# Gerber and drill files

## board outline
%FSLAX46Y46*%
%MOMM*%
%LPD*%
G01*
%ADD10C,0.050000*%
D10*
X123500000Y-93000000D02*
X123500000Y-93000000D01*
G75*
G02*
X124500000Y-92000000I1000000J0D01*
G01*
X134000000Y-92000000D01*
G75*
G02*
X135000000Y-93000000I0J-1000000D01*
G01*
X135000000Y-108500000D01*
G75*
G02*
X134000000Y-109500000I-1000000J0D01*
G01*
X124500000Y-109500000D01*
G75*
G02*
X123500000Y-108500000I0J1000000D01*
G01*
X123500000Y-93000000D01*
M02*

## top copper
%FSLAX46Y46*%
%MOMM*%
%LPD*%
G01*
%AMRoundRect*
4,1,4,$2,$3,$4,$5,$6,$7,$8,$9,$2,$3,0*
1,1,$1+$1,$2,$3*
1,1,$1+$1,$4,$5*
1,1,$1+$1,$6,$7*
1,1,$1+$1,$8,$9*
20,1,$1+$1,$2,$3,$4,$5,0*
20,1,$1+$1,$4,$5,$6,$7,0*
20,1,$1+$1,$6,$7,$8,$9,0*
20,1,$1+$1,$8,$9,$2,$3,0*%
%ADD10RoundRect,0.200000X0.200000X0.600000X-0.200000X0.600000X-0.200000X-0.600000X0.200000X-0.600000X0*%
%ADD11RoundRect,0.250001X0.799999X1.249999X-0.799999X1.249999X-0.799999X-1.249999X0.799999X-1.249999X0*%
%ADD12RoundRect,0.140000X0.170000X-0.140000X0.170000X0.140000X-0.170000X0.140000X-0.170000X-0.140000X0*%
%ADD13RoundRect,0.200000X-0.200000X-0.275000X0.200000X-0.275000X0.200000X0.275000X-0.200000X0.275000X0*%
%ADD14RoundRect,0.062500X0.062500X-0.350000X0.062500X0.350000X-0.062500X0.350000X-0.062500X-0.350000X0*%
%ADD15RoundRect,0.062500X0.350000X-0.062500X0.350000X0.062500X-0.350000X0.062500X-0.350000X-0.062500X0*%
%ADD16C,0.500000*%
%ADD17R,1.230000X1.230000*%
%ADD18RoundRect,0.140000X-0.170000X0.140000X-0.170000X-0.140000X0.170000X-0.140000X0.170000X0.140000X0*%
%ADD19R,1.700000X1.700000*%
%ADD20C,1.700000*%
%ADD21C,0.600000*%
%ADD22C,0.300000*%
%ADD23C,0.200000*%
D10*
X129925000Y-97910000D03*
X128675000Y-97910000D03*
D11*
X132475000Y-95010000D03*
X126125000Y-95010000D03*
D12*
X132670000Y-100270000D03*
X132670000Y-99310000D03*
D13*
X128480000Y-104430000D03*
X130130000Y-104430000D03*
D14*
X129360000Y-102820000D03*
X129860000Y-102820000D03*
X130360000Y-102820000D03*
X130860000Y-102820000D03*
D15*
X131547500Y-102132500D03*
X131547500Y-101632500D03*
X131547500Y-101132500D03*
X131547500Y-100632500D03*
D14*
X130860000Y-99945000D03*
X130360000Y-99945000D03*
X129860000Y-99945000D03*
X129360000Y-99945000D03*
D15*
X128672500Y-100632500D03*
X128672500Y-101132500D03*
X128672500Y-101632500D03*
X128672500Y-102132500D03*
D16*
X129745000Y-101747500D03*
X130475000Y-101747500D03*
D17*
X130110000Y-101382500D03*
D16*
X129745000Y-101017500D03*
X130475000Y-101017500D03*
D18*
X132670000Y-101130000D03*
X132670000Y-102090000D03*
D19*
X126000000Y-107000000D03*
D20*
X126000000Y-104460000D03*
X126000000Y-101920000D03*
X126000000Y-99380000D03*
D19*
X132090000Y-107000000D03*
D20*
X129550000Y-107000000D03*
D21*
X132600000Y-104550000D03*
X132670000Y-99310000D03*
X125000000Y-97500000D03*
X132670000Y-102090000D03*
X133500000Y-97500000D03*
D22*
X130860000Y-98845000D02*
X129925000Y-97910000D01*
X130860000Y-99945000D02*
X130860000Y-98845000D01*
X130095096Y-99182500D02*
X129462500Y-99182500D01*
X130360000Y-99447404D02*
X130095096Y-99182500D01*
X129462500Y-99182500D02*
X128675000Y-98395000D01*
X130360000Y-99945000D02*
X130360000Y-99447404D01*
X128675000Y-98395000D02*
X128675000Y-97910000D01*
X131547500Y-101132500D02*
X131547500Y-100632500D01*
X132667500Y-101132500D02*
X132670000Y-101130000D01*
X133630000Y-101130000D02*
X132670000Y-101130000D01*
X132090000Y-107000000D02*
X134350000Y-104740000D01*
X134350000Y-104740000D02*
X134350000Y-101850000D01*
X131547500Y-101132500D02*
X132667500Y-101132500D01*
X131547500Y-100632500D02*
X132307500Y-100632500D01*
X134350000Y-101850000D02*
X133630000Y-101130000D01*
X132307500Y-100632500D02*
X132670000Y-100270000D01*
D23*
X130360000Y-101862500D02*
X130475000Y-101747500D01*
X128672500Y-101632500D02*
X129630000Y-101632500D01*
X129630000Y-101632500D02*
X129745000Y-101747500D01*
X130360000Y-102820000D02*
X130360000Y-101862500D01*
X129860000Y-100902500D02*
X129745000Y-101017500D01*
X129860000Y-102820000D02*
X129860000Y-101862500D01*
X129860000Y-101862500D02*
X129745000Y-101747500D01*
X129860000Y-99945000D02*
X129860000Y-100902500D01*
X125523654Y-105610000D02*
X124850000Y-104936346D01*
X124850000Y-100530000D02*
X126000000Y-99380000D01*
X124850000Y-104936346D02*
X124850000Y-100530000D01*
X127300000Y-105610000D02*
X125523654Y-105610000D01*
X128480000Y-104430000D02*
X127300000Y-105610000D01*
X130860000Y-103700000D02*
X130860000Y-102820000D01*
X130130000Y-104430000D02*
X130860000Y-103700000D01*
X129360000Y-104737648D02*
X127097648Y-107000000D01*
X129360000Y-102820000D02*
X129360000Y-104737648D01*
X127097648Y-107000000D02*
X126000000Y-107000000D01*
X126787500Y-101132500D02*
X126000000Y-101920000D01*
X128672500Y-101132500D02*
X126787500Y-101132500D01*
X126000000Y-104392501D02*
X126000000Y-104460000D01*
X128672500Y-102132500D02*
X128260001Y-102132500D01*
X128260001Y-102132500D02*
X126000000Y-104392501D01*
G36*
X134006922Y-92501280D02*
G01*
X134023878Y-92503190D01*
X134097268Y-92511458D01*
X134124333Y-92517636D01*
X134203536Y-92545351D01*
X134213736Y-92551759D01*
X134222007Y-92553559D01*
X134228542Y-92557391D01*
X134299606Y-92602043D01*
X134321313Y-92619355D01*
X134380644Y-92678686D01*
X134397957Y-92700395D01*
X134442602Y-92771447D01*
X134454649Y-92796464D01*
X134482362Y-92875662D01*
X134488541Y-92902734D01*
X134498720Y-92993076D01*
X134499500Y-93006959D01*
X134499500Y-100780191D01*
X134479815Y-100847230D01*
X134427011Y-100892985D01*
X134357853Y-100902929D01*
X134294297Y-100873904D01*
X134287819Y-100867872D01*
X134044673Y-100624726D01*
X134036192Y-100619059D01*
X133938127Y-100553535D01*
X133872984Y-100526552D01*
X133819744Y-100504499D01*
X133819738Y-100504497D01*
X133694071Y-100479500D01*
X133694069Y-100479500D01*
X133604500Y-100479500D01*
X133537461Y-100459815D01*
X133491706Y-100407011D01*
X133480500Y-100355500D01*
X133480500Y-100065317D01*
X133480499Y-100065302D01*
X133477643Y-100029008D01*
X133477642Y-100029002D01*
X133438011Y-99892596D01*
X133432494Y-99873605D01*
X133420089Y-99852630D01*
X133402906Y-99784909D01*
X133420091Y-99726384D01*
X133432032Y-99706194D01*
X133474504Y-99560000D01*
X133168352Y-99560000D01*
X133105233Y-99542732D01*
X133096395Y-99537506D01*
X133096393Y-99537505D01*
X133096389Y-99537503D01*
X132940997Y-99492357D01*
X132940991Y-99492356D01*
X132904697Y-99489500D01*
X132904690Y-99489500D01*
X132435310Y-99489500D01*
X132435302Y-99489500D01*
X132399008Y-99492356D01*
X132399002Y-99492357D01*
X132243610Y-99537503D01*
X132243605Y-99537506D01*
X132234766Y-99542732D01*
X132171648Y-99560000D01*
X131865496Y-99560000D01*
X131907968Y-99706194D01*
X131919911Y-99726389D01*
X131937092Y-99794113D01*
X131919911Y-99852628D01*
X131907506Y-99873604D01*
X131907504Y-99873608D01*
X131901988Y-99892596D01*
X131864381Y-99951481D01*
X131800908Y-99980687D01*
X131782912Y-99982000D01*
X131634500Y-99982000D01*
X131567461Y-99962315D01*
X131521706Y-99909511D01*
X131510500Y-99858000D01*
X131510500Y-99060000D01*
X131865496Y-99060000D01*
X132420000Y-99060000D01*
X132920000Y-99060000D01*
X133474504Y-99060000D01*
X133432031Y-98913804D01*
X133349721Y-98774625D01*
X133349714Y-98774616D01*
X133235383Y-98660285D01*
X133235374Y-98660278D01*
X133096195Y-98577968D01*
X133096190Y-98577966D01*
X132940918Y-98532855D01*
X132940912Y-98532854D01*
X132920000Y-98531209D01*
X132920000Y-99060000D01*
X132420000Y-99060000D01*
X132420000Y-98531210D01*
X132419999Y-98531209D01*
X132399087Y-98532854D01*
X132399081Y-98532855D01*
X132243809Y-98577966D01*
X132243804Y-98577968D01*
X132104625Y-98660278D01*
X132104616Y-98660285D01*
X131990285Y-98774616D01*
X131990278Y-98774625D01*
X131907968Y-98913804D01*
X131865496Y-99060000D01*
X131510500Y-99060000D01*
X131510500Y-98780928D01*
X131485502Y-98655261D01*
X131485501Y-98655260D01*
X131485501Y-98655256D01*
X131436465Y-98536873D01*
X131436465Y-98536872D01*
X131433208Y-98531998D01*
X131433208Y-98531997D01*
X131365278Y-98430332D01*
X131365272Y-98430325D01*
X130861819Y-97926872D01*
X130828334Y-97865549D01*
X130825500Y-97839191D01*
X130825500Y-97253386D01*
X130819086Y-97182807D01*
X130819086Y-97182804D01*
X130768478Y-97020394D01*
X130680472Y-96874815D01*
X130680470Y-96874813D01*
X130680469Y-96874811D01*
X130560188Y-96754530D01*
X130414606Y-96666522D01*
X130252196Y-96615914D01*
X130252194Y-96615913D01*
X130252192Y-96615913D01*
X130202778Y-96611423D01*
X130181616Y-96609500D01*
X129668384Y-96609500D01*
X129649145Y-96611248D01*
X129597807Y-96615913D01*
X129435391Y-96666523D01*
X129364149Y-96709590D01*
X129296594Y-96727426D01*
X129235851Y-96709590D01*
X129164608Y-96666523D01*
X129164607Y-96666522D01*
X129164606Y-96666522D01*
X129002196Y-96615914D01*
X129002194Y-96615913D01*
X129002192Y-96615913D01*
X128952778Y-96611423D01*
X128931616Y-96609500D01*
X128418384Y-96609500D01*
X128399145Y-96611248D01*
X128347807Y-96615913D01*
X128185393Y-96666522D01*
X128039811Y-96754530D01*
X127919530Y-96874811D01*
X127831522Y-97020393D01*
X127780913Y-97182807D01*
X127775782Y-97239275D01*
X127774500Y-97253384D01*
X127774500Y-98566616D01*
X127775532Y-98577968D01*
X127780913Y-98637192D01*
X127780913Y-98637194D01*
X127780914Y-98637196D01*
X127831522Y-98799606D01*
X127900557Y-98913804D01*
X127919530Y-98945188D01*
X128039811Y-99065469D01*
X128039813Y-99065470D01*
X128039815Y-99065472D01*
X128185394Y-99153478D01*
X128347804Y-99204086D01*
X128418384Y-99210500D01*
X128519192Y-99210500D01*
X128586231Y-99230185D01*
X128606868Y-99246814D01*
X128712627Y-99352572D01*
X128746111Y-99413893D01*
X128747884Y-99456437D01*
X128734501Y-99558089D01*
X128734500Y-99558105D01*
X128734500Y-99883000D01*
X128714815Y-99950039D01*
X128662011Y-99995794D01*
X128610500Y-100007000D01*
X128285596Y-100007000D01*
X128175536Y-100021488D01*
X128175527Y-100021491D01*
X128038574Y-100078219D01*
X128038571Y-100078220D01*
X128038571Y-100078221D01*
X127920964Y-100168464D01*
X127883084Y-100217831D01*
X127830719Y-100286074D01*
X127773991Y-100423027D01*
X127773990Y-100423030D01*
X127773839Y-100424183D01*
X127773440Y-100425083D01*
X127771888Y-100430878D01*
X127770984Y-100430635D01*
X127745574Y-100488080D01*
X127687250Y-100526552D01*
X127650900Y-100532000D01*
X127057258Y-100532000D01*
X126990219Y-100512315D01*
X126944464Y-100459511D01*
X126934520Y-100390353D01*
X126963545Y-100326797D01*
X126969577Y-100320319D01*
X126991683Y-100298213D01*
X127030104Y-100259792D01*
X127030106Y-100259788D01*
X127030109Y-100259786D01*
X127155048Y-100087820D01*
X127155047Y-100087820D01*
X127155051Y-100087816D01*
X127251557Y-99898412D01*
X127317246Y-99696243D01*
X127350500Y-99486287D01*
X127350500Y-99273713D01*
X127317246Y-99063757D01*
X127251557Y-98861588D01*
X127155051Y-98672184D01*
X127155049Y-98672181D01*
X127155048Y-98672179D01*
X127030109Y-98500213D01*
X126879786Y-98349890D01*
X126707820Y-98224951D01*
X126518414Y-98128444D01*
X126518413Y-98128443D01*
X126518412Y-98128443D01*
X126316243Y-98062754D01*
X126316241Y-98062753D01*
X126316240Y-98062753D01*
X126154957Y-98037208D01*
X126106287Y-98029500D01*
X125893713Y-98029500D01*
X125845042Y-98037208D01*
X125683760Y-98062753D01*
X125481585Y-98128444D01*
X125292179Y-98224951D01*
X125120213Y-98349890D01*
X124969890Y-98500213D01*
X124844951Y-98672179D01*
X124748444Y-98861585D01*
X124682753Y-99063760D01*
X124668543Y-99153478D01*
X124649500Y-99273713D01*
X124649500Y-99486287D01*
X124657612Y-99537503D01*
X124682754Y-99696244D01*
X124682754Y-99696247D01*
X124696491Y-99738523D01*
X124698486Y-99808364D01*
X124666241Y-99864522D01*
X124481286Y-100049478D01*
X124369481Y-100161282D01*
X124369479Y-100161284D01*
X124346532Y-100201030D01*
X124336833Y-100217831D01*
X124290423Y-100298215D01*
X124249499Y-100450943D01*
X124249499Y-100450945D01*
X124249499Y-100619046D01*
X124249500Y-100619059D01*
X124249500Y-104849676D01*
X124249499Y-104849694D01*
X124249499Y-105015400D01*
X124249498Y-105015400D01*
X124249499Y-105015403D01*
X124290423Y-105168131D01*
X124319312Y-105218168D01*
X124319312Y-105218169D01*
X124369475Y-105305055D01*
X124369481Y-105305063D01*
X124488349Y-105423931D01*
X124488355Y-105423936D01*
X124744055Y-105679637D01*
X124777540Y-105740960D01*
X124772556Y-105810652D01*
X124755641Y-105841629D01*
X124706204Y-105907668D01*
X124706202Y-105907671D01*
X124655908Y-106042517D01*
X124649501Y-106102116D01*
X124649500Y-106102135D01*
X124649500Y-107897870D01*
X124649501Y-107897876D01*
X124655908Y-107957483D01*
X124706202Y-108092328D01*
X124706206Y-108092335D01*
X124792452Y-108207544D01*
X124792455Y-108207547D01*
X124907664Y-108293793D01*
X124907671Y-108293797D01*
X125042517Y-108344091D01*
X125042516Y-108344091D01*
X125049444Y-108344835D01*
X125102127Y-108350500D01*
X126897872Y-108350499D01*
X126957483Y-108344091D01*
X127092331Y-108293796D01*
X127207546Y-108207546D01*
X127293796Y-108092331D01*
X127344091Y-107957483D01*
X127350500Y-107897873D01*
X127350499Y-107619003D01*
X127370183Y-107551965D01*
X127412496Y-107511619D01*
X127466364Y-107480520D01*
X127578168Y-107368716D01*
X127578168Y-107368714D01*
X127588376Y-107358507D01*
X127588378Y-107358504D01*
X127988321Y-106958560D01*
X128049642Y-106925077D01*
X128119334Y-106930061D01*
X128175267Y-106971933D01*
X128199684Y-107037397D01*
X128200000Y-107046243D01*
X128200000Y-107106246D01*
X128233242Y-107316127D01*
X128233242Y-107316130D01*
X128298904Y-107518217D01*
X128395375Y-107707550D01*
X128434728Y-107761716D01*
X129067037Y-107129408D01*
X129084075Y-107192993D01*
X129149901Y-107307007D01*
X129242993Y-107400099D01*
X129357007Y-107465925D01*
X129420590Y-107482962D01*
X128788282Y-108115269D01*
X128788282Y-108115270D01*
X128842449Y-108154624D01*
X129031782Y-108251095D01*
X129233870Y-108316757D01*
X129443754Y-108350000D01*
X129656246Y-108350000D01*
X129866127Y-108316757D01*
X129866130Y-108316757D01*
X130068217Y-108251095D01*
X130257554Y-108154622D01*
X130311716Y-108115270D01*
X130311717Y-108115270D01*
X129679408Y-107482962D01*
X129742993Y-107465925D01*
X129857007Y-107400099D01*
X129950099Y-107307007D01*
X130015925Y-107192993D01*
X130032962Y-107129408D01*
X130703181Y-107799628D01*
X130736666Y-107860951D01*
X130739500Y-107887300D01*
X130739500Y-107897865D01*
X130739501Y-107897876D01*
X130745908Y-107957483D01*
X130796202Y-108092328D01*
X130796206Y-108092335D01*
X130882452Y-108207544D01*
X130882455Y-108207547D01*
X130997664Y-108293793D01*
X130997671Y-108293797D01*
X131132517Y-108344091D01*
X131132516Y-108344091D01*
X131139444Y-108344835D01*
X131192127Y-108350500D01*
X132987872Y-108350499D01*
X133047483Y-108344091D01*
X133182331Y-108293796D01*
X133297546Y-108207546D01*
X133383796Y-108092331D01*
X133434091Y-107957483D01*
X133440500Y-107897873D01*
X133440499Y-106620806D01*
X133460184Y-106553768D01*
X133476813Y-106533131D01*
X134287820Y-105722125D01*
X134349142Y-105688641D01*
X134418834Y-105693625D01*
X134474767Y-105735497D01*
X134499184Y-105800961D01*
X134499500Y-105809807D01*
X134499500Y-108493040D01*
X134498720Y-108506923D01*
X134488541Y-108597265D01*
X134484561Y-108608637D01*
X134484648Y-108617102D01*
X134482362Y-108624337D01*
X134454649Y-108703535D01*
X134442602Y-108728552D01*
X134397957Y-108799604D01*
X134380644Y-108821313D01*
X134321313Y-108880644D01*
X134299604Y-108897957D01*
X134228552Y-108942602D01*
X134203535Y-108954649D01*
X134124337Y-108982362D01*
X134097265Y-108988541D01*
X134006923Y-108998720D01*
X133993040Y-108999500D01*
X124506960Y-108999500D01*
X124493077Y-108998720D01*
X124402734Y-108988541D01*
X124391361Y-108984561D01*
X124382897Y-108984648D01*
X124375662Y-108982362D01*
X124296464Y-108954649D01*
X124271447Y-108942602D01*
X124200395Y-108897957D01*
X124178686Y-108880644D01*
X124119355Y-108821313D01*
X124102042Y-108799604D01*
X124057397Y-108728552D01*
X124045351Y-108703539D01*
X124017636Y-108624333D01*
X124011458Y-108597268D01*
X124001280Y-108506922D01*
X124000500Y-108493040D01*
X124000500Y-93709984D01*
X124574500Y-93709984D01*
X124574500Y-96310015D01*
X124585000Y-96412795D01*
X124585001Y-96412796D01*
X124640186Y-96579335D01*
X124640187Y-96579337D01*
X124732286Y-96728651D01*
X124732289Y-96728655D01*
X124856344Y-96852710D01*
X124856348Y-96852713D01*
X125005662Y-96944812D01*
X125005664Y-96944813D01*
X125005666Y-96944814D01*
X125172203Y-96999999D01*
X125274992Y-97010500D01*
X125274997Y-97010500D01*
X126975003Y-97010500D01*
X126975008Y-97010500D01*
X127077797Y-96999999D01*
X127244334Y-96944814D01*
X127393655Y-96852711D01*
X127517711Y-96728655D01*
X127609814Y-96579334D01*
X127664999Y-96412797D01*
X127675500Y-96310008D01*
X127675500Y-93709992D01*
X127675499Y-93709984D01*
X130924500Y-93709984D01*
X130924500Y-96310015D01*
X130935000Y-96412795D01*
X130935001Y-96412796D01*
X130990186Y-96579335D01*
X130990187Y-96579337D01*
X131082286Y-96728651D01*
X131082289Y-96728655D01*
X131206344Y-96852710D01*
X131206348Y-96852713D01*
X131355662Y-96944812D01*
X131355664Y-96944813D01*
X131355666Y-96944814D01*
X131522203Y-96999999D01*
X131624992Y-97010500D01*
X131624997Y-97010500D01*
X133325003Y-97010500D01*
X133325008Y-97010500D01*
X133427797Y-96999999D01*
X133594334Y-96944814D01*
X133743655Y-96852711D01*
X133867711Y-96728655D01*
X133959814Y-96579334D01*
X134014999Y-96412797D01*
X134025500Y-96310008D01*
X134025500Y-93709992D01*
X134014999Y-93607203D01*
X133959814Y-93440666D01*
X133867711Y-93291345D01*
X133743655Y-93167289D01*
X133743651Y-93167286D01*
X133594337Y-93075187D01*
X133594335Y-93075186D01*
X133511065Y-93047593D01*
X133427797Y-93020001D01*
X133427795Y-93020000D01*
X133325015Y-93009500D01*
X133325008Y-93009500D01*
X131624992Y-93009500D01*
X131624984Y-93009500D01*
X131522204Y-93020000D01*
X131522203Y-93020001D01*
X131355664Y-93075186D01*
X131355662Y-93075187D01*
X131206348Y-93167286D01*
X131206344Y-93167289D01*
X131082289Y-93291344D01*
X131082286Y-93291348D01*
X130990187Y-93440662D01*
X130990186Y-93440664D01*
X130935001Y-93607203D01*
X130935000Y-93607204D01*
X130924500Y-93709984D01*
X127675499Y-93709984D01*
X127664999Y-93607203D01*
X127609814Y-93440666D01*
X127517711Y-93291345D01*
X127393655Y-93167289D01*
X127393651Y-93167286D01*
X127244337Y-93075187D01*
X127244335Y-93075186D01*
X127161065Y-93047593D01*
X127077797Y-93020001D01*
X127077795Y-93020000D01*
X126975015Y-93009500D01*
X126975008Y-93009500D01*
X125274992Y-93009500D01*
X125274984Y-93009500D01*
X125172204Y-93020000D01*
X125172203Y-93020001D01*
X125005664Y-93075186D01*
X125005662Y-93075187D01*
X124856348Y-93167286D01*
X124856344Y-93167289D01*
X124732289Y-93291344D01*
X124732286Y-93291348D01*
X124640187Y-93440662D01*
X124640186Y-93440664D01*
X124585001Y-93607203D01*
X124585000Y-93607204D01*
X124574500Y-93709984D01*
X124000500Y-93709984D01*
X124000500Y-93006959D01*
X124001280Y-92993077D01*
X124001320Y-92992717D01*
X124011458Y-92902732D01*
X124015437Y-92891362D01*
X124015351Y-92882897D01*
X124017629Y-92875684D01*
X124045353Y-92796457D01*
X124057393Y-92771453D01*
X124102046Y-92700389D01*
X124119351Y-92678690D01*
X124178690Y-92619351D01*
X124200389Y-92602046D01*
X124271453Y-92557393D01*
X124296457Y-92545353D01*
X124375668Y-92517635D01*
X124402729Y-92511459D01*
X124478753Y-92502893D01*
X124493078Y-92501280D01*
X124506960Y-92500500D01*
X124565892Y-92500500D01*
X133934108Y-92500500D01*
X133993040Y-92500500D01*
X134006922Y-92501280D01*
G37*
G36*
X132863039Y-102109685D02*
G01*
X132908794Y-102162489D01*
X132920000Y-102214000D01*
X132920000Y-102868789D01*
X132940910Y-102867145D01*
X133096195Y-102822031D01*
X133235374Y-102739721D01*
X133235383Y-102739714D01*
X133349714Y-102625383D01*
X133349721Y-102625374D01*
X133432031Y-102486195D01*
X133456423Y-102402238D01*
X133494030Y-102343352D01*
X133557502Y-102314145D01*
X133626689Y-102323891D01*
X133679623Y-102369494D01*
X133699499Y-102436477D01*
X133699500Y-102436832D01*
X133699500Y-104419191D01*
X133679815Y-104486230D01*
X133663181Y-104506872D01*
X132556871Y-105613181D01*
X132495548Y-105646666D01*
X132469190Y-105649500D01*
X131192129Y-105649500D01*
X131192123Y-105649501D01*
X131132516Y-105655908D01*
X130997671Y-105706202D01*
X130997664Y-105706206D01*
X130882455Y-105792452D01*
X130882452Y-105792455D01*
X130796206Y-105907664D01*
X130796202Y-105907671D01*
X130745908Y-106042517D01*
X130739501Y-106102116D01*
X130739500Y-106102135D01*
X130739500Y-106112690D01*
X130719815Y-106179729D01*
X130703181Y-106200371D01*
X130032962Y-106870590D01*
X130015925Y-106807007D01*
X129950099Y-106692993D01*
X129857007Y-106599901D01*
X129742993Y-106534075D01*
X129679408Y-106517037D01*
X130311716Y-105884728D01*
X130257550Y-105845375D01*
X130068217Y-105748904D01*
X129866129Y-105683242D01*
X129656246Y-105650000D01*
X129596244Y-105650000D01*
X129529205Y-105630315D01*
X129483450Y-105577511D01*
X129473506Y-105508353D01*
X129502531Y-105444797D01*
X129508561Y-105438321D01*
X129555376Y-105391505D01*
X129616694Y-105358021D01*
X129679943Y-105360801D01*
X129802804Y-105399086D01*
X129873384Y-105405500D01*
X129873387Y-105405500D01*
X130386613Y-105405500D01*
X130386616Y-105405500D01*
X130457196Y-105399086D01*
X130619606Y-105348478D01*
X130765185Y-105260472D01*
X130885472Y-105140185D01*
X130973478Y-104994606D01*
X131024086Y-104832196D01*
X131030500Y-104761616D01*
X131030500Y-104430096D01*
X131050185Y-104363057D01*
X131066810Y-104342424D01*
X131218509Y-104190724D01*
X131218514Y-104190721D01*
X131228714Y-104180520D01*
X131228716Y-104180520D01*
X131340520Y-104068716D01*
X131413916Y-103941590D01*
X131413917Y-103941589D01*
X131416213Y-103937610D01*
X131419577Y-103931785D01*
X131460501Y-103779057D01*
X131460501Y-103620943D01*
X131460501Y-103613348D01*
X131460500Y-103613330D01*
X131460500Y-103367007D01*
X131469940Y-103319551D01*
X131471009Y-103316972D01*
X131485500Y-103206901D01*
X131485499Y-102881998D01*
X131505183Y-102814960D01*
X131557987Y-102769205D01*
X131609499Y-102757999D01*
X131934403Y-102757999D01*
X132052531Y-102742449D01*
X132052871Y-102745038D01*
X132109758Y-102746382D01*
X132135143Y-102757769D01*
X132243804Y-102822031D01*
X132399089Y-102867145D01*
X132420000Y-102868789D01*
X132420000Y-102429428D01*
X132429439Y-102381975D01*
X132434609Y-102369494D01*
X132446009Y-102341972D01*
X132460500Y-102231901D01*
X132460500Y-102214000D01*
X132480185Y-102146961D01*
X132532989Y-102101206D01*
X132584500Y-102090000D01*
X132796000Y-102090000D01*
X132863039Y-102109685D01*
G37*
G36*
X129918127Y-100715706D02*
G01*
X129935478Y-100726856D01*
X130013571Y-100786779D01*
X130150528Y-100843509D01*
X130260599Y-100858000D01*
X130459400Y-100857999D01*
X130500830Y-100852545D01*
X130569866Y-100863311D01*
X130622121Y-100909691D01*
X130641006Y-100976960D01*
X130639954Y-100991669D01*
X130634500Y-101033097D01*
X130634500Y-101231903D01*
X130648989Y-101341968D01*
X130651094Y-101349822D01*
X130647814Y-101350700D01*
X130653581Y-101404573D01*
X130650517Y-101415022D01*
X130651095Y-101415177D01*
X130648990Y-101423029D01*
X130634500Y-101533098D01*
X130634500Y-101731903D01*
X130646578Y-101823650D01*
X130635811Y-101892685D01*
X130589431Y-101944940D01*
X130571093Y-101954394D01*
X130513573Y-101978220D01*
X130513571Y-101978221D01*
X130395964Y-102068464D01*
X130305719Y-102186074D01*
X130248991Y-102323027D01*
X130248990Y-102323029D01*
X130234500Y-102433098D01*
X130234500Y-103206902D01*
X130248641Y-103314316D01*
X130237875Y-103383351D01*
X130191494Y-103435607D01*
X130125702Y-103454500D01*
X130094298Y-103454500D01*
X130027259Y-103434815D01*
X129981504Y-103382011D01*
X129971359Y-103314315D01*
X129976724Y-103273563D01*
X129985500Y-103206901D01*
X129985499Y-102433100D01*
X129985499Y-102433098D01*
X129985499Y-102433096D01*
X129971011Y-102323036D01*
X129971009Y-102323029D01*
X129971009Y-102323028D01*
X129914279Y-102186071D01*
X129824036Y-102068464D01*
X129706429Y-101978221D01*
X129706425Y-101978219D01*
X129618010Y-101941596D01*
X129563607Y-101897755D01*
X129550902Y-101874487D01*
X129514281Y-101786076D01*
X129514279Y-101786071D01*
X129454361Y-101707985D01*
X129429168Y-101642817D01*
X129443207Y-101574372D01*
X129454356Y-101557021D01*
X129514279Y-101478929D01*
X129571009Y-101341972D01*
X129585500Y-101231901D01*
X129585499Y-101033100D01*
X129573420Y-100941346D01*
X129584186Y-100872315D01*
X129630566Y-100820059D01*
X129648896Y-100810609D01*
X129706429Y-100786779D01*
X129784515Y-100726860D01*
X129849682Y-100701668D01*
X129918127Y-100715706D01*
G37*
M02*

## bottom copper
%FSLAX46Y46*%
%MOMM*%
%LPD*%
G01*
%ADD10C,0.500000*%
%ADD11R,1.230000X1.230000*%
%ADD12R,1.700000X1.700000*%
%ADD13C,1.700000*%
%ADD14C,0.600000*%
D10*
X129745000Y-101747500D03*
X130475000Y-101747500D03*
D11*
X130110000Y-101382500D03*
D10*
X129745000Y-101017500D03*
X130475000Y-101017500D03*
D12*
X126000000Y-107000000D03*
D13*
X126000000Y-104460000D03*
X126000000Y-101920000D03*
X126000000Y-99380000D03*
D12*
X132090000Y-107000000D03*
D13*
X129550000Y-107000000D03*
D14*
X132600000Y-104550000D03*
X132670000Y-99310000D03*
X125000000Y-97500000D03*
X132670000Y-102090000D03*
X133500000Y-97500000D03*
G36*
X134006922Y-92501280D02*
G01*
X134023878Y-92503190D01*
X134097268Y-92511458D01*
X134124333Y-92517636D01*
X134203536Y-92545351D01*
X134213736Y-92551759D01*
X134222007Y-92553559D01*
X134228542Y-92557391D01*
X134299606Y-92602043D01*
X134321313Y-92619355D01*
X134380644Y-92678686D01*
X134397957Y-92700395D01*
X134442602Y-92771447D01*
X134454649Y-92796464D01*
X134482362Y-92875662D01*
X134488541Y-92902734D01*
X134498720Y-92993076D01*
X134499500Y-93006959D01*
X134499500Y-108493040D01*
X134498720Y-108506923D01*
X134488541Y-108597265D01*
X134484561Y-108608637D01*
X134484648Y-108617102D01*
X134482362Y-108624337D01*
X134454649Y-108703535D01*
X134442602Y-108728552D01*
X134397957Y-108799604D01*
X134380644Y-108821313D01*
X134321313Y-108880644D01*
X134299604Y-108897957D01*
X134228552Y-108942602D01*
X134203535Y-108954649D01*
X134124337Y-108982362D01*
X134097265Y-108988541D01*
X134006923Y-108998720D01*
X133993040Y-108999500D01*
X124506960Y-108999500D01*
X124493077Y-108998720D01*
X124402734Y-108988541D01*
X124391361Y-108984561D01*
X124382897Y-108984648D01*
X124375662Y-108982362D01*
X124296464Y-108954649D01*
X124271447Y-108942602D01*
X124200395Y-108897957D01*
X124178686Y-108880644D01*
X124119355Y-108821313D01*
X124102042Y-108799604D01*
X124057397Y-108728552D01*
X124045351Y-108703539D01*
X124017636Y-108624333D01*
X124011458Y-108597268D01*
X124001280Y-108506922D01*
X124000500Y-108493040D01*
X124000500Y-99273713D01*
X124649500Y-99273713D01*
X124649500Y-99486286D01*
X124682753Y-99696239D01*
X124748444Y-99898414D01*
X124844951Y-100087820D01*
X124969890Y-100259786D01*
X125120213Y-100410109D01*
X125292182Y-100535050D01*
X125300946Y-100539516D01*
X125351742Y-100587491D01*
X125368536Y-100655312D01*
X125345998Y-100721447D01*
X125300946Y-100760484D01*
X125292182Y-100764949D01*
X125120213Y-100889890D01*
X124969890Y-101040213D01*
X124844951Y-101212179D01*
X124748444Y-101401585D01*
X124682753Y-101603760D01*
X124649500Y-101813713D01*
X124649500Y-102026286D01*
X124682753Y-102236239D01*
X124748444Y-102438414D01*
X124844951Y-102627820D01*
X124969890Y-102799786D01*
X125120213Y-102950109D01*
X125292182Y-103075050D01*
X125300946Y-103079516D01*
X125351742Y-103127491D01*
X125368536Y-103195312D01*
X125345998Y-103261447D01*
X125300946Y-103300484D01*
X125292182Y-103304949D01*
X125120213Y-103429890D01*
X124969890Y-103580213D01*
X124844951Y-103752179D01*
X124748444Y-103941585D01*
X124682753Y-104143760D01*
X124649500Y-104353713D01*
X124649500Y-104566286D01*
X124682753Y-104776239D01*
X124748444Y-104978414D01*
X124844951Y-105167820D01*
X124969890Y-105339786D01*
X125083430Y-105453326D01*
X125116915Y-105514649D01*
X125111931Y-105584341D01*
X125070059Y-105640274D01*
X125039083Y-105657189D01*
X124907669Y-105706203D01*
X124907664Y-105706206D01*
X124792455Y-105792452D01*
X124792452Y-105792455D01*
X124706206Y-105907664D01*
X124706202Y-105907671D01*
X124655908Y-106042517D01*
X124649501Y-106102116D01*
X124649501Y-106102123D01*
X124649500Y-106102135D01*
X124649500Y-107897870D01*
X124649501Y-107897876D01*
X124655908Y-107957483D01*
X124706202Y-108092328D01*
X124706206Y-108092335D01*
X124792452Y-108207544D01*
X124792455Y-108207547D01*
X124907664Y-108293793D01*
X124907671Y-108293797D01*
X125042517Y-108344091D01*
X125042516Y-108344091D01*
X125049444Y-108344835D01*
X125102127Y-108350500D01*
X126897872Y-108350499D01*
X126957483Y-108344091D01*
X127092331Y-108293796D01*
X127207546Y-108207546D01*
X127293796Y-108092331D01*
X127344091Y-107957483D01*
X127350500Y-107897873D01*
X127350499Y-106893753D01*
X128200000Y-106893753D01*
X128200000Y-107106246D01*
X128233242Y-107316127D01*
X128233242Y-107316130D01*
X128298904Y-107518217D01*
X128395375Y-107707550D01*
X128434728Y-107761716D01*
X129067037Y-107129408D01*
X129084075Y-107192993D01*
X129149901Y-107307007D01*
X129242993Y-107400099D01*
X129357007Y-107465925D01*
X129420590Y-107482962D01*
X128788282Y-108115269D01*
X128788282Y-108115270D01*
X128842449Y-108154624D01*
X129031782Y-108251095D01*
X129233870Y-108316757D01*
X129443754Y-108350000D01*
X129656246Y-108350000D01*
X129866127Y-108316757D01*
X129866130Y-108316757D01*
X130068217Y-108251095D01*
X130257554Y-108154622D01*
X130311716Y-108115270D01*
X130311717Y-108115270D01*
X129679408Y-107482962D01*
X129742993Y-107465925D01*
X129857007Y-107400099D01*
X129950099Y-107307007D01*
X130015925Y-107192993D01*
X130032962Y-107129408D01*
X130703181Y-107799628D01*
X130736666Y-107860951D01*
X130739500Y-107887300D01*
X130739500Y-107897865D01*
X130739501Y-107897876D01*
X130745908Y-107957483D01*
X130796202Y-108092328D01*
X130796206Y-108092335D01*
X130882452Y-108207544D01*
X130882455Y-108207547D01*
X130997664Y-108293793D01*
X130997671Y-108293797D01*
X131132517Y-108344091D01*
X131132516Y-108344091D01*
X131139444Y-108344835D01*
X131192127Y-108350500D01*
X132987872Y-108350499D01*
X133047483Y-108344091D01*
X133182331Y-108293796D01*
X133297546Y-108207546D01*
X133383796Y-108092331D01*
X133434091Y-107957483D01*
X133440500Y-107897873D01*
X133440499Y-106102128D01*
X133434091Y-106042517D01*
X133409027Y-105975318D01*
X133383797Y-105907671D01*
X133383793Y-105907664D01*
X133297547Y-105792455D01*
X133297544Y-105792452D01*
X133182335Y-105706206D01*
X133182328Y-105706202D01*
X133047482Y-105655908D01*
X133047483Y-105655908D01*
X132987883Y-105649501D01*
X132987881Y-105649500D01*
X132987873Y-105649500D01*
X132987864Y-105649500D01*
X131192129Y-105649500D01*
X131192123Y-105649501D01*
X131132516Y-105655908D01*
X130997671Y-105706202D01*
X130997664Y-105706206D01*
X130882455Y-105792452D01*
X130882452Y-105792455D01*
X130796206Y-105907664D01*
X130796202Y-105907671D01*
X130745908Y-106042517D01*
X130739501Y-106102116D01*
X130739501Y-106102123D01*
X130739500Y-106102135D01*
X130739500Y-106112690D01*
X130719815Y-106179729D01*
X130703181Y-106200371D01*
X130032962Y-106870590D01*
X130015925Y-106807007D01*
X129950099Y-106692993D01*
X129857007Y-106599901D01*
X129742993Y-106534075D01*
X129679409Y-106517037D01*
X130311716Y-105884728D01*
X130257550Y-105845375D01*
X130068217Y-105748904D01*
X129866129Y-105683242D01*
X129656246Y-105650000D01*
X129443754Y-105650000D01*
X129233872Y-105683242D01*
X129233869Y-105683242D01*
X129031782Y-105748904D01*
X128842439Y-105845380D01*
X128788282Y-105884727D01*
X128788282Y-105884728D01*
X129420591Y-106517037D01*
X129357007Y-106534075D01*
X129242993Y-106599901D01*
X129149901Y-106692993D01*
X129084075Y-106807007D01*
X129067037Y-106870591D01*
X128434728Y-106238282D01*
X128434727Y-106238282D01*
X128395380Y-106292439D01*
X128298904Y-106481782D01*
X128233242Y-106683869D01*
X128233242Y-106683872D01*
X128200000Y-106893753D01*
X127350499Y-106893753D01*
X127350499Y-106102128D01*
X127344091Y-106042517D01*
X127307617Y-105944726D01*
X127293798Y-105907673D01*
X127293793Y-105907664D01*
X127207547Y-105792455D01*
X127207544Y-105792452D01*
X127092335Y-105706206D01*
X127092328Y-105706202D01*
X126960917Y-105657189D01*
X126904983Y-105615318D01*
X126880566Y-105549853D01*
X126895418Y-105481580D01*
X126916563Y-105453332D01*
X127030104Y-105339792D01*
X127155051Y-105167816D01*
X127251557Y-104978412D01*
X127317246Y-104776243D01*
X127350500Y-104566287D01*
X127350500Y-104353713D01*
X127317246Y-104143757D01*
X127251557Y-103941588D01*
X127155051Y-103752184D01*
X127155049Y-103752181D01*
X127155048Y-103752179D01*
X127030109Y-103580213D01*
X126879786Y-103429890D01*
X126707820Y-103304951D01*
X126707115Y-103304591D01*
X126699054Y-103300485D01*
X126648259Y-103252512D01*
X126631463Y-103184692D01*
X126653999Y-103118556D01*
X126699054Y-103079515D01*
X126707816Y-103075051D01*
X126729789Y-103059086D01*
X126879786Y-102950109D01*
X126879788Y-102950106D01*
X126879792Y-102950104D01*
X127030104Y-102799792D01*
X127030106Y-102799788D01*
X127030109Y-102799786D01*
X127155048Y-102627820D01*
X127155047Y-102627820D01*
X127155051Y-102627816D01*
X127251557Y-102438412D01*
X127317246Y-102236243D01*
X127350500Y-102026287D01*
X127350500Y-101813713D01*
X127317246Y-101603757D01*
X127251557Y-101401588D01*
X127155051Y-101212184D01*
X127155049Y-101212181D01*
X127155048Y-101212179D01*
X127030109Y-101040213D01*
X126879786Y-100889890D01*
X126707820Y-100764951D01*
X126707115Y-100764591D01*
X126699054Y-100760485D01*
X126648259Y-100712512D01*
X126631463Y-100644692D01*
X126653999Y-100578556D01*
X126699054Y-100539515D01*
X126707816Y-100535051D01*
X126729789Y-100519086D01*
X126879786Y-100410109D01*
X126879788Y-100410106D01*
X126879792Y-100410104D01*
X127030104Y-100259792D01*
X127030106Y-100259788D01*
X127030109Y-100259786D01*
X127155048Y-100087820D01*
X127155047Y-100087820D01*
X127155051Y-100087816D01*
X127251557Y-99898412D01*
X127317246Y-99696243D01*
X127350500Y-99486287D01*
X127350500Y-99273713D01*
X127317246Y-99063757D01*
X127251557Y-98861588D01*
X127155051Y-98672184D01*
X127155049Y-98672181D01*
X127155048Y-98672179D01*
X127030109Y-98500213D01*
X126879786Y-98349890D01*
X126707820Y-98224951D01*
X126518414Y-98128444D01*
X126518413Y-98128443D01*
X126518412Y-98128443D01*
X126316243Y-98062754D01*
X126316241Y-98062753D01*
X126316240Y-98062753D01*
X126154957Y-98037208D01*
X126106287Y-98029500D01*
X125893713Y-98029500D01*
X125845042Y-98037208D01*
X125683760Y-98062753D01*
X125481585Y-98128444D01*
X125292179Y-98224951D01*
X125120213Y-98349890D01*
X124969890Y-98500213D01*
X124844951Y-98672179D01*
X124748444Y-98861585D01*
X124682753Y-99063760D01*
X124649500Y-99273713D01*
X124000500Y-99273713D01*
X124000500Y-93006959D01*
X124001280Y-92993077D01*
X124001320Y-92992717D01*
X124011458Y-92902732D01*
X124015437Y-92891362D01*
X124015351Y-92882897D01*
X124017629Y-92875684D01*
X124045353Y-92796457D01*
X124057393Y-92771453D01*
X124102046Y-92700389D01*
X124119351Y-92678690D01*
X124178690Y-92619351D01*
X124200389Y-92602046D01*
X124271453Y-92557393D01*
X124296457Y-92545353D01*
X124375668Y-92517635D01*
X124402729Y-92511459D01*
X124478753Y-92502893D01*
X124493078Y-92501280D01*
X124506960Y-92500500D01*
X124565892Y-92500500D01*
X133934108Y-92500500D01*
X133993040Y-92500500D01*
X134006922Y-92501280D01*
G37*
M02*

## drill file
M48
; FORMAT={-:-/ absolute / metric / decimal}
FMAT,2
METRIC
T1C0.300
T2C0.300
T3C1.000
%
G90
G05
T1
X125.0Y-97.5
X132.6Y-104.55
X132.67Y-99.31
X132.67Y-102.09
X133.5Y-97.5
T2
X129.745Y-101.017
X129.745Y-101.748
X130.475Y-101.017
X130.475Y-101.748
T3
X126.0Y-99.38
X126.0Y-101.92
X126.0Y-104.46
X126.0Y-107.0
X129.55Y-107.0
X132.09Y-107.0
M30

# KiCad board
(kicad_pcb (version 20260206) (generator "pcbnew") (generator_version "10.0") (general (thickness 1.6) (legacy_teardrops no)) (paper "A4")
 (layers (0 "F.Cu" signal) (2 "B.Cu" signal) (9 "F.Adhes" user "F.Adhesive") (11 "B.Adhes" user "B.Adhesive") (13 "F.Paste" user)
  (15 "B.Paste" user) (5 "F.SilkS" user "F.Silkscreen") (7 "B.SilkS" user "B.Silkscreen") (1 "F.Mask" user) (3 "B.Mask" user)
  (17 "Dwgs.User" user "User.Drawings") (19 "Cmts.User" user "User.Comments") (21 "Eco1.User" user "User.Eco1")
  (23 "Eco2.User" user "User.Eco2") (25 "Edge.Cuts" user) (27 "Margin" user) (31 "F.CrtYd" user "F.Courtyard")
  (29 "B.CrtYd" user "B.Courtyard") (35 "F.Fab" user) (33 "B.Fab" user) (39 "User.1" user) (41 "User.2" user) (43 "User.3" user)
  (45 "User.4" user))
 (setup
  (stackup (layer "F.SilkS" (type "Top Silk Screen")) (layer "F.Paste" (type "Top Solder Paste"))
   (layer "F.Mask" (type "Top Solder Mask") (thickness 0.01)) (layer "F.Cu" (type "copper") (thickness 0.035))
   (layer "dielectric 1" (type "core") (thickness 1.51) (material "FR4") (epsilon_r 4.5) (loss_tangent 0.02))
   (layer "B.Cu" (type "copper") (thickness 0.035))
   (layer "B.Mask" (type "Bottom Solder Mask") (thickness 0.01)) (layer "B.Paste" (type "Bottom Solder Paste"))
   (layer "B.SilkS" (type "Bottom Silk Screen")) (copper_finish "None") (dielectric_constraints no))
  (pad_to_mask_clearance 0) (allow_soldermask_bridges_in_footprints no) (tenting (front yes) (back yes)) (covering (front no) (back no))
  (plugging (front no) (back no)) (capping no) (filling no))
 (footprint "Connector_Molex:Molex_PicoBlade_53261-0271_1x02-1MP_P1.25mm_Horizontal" (layer "F.Cu") (at 129.3 95.51 180)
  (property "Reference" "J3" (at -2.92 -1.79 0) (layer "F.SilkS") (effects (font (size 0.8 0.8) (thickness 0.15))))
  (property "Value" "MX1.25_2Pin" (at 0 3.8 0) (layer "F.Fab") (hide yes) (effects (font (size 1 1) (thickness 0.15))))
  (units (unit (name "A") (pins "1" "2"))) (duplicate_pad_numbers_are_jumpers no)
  (pad "1" smd roundrect (at -0.625 -2.4 180) (size 0.8 1.6) (layers "F.Cu" "F.Mask" "F.Paste") (roundrect_rratio 0.25)
   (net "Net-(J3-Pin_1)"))
  (pad "2" smd roundrect (at 0.625 -2.4 180) (size 0.8 1.6) (layers "F.Cu" "F.Mask" "F.Paste") (roundrect_rratio 0.25)
   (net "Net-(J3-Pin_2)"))
  (pad "MP" smd roundrect (at -3.175 0.5 180) (size 2.1 3) (layers "F.Cu" "F.Mask" "F.Paste") (roundrect_rratio 0.119048))
  (pad "MP" smd roundrect (at 3.175 0.5 180) (size 2.1 3) (layers "F.Cu" "F.Mask" "F.Paste") (roundrect_rratio 0.119048)))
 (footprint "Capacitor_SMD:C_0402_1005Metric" (layer "F.Cu") (at 132.67 99.79 90)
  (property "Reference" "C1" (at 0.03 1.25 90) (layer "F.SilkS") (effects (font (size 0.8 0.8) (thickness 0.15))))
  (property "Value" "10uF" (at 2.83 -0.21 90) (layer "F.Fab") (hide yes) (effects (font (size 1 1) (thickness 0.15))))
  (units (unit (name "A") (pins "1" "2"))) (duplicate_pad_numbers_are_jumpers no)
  (pad "1" smd roundrect (at -0.48 0 90) (size 0.56 0.62) (layers "F.Cu" "F.Mask" "F.Paste") (roundrect_rratio 0.25) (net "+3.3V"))
  (pad "2" smd roundrect (at 0.48 0 90) (size 0.56 0.62) (layers "F.Cu" "F.Mask" "F.Paste") (roundrect_rratio 0.25) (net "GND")))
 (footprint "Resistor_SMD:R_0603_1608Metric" (layer "F.Cu") (at 129.305 104.43)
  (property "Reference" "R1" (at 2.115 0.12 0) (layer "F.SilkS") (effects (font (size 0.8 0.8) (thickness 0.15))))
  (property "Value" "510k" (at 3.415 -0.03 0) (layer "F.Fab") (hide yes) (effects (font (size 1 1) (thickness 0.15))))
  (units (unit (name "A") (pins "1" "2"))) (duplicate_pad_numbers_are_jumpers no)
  (pad "1" smd roundrect (at -0.825 0) (size 0.8 0.95) (layers "F.Cu" "F.Mask" "F.Paste") (roundrect_rratio 0.25) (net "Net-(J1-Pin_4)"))
  (pad "2" smd roundrect (at 0.825 0) (size 0.8 0.95) (layers "F.Cu" "F.Mask" "F.Paste") (roundrect_rratio 0.25) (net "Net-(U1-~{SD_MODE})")))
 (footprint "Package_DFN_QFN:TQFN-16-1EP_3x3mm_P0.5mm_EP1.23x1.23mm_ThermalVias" (layer "F.Cu") (at 130.11 101.3825 90)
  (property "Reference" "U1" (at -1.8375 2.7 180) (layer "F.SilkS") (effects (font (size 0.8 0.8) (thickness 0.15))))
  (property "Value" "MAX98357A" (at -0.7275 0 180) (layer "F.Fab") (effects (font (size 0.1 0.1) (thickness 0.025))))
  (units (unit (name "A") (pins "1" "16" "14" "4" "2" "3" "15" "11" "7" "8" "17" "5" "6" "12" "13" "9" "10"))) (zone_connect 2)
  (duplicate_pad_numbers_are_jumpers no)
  (pad "" smd roundrect (at -0.31 -0.31 90) (size 0.53 0.53) (layers "F.Paste") (roundrect_rratio 0.25))
  (pad "" smd roundrect (at -0.31 0.31 90) (size 0.53 0.53) (layers "F.Paste") (roundrect_rratio 0.25))
  (pad "" smd roundrect (at 0.31 -0.31 90) (size 0.53 0.53) (layers "F.Paste") (roundrect_rratio 0.25))
  (pad "" smd roundrect (at 0.31 0.31 90) (size 0.53 0.53) (layers "F.Paste") (roundrect_rratio 0.25))
  (pad "1" smd roundrect (at -1.4375 -0.75 90) (size 0.825 0.25) (layers "F.Cu" "F.Mask" "F.Paste") (roundrect_rratio 0.25)
   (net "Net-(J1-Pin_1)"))
  (pad "2" smd roundrect (at -1.4375 -0.25 90) (size 0.825 0.25) (layers "F.Cu" "F.Mask" "F.Paste") (roundrect_rratio 0.25) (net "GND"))
  (pad "3" smd roundrect (at -1.4375 0.25 90) (size 0.825 0.25) (layers "F.Cu" "F.Mask" "F.Paste") (roundrect_rratio 0.25) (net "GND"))
  (pad "4" smd roundrect (at -1.4375 0.75 90) (size 0.825 0.25) (layers "F.Cu" "F.Mask" "F.Paste") (roundrect_rratio 0.25)
   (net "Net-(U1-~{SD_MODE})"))
  (pad "5" smd roundrect (at -0.75 1.4375 90) (size 0.25 0.825) (layers "F.Cu" "F.Mask" "F.Paste") (roundrect_rratio 0.25)
   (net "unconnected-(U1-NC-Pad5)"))
  (pad "6" smd roundrect (at -0.25 1.4375 90) (size 0.25 0.825) (layers "F.Cu" "F.Mask" "F.Paste") (roundrect_rratio 0.25)
   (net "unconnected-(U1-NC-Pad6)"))
  (pad "7" smd roundrect (at 0.25 1.4375 90) (size 0.25 0.825) (layers "F.Cu" "F.Mask" "F.Paste") (roundrect_rratio 0.25) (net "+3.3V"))
  (pad "8" smd roundrect (at 0.75 1.4375 90) (size 0.25 0.825) (layers "F.Cu" "F.Mask" "F.Paste") (roundrect_rratio 0.25) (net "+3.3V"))
  (pad "9" smd roundrect (at 1.4375 0.75 90) (size 0.825 0.25) (layers "F.Cu" "F.Mask" "F.Paste") (roundrect_rratio 0.25)
   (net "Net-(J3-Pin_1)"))
  (pad "10" smd roundrect (at 1.4375 0.25 90) (size 0.825 0.25) (layers "F.Cu" "F.Mask" "F.Paste") (roundrect_rratio 0.25)
   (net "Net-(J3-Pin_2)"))
  (pad "11" smd roundrect (at 1.4375 -0.25 90) (size 0.825 0.25) (layers "F.Cu" "F.Mask" "F.Paste") (roundrect_rratio 0.25) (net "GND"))
  (pad "12" smd roundrect (at 1.4375 -0.75 90) (size 0.825 0.25) (layers "F.Cu" "F.Mask" "F.Paste") (roundrect_rratio 0.25)
   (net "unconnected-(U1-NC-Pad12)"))
  (pad "13" smd roundrect (at 0.75 -1.4375 90) (size 0.25 0.825) (layers "F.Cu" "F.Mask" "F.Paste") (roundrect_rratio 0.25)
   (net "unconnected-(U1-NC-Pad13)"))
  (pad "14" smd roundrect (at 0.25 -1.4375 90) (size 0.25 0.825) (layers "F.Cu" "F.Mask" "F.Paste") (roundrect_rratio 0.25)
   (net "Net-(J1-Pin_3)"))
  (pad "15" smd roundrect (at -0.25 -1.4375 90) (size 0.25 0.825) (layers "F.Cu" "F.Mask" "F.Paste") (roundrect_rratio 0.25) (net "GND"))
  (pad "16" smd roundrect (at -0.75 -1.4375 90) (size 0.25 0.825) (layers "F.Cu" "F.Mask" "F.Paste") (roundrect_rratio 0.25)
   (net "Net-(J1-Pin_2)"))
  (pad "17" thru_hole circle (at -0.365 -0.365 90) (size 0.5 0.5) (drill 0.3) (layers "*.Cu") (remove_unused_layers no) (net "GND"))
  (pad "17" thru_hole circle (at -0.365 0.365 90) (size 0.5 0.5) (drill 0.3) (layers "*.Cu") (remove_unused_layers no) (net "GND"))
  (pad "17" smd rect (at 0 0 90) (size 1.23 1.23) (layers "F.Cu" "F.Mask") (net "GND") (zone_connect 2))
  (pad "17" smd rect (at 0 0 90) (size 1.23 1.23) (layers "B.Cu") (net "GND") (zone_connect 2))
  (pad "17" thru_hole circle (at 0.365 -0.365 90) (size 0.5 0.5) (drill 0.3) (layers "*.Cu") (remove_unused_layers no) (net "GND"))
  (pad "17" thru_hole circle (at 0.365 0.365 90) (size 0.5 0.5) (drill 0.3) (layers "*.Cu") (remove_unused_layers no) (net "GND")))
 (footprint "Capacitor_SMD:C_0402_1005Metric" (layer "F.Cu") (at 132.67 101.61 -90)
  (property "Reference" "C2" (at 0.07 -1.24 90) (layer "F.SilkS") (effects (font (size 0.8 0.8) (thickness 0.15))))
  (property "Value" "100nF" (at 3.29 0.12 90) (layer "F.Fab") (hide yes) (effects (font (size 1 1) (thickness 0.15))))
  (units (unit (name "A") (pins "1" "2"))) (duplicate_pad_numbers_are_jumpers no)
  (pad "1" smd roundrect (at -0.48 0 270) (size 0.56 0.62) (layers "F.Cu" "F.Mask" "F.Paste") (roundrect_rratio 0.25) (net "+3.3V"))
  (pad "2" smd roundrect (at 0.48 0 270) (size 0.56 0.62) (layers "F.Cu" "F.Mask" "F.Paste") (roundrect_rratio 0.25) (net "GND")))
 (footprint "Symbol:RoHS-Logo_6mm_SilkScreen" (layer "B.Cu") (at 125.5 95 -90)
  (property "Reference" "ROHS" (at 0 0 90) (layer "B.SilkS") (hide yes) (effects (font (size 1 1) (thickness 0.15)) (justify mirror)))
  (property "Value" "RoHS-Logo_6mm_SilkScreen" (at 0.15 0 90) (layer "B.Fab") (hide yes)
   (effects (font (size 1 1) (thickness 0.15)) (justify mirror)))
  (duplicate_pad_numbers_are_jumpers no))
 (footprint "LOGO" (layer "B.Cu") (at 129 97.25 -90)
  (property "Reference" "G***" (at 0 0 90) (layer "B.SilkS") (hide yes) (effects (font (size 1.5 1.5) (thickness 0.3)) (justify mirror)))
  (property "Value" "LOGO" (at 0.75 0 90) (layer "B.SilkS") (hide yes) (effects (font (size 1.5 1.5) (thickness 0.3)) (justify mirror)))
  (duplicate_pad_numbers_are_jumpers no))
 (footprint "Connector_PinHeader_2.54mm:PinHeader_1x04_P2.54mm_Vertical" (layer "B.Cu") (at 126 107)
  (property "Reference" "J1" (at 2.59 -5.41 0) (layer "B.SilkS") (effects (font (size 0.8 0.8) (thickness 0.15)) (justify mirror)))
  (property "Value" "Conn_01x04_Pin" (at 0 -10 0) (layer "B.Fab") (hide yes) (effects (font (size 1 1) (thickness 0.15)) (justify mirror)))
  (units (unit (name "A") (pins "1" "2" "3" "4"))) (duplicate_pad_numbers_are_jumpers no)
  (pad "1" thru_hole rect (at 0 0) (size 1.7 1.7) (drill 1) (layers "*.Cu" "*.Mask") (remove_unused_layers no) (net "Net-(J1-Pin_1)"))
  (pad "2" thru_hole circle (at 0 -2.54) (size 1.7 1.7) (drill 1) (layers "*.Cu" "*.Mask") (remove_unused_layers no) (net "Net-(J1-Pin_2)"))
  (pad "3" thru_hole circle (at 0 -5.08) (size 1.7 1.7) (drill 1) (layers "*.Cu" "*.Mask") (remove_unused_layers no) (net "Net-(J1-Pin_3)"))
  (pad "4" thru_hole circle (at 0 -7.62) (size 1.7 1.7) (drill 1) (layers "*.Cu" "*.Mask") (remove_unused_layers no) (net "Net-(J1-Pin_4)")))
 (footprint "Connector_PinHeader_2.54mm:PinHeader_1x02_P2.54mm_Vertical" (layer "B.Cu") (at 132.09 107 90)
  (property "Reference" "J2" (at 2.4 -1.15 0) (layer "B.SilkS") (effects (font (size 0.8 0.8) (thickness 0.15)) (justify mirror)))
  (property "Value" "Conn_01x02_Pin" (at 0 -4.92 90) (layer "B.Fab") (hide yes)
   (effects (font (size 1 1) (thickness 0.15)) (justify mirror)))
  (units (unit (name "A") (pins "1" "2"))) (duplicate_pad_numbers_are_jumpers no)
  (pad "1" thru_hole rect (at 0 0 90) (size 1.7 1.7) (drill 1) (layers "*.Cu" "*.Mask") (remove_unused_layers no) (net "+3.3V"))
  (pad "2" thru_hole circle (at 0 -2.54 90) (size 1.7 1.7) (drill 1) (layers "*.Cu" "*.Mask") (remove_unused_layers no) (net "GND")))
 (gr_rect (start 123.5 92) (end 135 109.5) (radius 1) (stroke (width 0.05) (type default)) (fill no) (layer "Edge.Cuts"))
 (segment (start 130.86 98.845) (end 129.925 97.91) (width 0.3) (layer "F.Cu") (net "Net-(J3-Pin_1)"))
 (segment (start 130.86 99.945) (end 130.86 98.845) (width 0.3) (layer "F.Cu") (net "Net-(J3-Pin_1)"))
 (segment (start 130.095096 99.1825) (end 129.4625 99.1825) (width 0.3) (layer "F.Cu") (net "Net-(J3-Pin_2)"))
 (segment (start 130.36 99.447404) (end 130.095096 99.1825) (width 0.3) (layer "F.Cu") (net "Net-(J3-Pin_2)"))
 (segment (start 129.4625 99.1825) (end 128.675 98.395) (width 0.3) (layer "F.Cu") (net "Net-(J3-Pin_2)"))
 (segment (start 130.36 99.945) (end 130.36 99.447404) (width 0.3) (layer "F.Cu") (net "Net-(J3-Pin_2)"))
 (segment (start 128.675 98.395) (end 128.675 97.91) (width 0.3) (layer "F.Cu") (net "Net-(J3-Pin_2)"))
 (segment (start 131.5475 101.1325) (end 131.5475 100.6325) (width 0.3) (layer "F.Cu") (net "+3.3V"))
 (segment (start 132.6675 101.1325) (end 132.67 101.13) (width 0.3) (layer "F.Cu") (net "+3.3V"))
 (segment (start 133.63 101.13) (end 132.67 101.13) (width 0.3) (layer "F.Cu") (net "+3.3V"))
 (segment (start 132.09 107) (end 134.35 104.74) (width 0.3) (layer "F.Cu") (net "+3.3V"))
 (segment (start 134.35 104.74) (end 134.35 101.85) (width 0.3) (layer "F.Cu") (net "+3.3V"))
 (segment (start 131.5475 101.1325) (end 132.6675 101.1325) (width 0.3) (layer "F.Cu") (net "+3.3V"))
 (segment (start 131.5475 100.6325) (end 132.3075 100.6325) (width 0.3) (layer "F.Cu") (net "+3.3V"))
 (segment (start 134.35 101.85) (end 133.63 101.13) (width 0.3) (layer "F.Cu") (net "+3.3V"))
 (segment (start 132.3075 100.6325) (end 132.67 100.27) (width 0.3) (layer "F.Cu") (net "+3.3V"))
 (segment (start 130.36 101.8625) (end 130.475 101.7475) (width 0.2) (layer "F.Cu") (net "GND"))
 (segment (start 128.6725 101.6325) (end 129.63 101.6325) (width 0.2) (layer "F.Cu") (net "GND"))
 (segment (start 129.63 101.6325) (end 129.745 101.7475) (width 0.2) (layer "F.Cu") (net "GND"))
 (segment (start 130.36 102.82) (end 130.36 101.8625) (width 0.2) (layer "F.Cu") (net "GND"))
 (segment (start 129.86 100.9025) (end 129.745 101.0175) (width 0.2) (layer "F.Cu") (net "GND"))
 (segment (start 129.86 102.82) (end 129.86 101.8625) (width 0.2) (layer "F.Cu") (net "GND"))
 (segment (start 129.86 101.8625) (end 129.745 101.7475) (width 0.2) (layer "F.Cu") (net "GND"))
 (segment (start 129.86 99.945) (end 129.86 100.9025) (width 0.2) (layer "F.Cu") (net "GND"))
 (via (at 132.6 104.55) (size 0.6) (drill 0.3) (layers "F.Cu" "B.Cu") (free yes) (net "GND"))
 (via (at 132.67 99.31) (size 0.6) (drill 0.3) (layers "F.Cu" "B.Cu") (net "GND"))
 (via (at 125 97.5) (size 0.6) (drill 0.3) (layers "F.Cu" "B.Cu") (free yes) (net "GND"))
 (via (at 132.67 102.09) (size 0.6) (drill 0.3) (layers "F.Cu" "B.Cu") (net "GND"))
 (via (at 133.5 97.5) (size 0.6) (drill 0.3) (layers "F.Cu" "B.Cu") (free yes) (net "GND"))
 (segment (start 125.523654 105.61) (end 124.85 104.936346) (width 0.2) (layer "F.Cu") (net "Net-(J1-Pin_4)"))
 (segment (start 124.85 100.53) (end 126 99.38) (width 0.2) (layer "F.Cu") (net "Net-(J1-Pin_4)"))
 (segment (start 124.85 104.936346) (end 124.85 100.53) (width 0.2) (layer "F.Cu") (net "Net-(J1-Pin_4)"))
 (segment (start 127.3 105.61) (end 125.523654 105.61) (width 0.2) (layer "F.Cu") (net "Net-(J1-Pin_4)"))
 (segment (start 128.48 104.43) (end 127.3 105.61) (width 0.2) (layer "F.Cu") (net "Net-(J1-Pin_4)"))
 (segment (start 130.86 103.7) (end 130.86 102.82) (width 0.2) (layer "F.Cu") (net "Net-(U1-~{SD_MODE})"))
 (segment (start 130.13 104.43) (end 130.86 103.7) (width 0.2) (layer "F.Cu") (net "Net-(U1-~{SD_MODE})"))
 (segment (start 129.36 104.737648) (end 127.097648 107) (width 0.2) (layer "F.Cu") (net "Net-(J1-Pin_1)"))
 (segment (start 129.36 102.82) (end 129.36 104.737648) (width 0.2) (layer "F.Cu") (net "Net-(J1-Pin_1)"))
 (segment (start 127.097648 107) (end 126 107) (width 0.2) (layer "F.Cu") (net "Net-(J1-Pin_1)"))
 (segment (start 126.7875 101.1325) (end 126 101.92) (width 0.2) (layer "F.Cu") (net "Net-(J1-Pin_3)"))
 (segment (start 128.6725 101.1325) (end 126.7875 101.1325) (width 0.2) (layer "F.Cu") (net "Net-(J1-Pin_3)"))
 (segment (start 126 104.392501) (end 126 104.46) (width 0.2) (layer "F.Cu") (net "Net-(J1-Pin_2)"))
 (segment (start 128.6725 102.1325) (end 128.260001 102.1325) (width 0.2) (layer "F.Cu") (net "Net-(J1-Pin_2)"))
 (segment (start 128.260001 102.1325) (end 126 104.392501) (width 0.2) (layer "F.Cu") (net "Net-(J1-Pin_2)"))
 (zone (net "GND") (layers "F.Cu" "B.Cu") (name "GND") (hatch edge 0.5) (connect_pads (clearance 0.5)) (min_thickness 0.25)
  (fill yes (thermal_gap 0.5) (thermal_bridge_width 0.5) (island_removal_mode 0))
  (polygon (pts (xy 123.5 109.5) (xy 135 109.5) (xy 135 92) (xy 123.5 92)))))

